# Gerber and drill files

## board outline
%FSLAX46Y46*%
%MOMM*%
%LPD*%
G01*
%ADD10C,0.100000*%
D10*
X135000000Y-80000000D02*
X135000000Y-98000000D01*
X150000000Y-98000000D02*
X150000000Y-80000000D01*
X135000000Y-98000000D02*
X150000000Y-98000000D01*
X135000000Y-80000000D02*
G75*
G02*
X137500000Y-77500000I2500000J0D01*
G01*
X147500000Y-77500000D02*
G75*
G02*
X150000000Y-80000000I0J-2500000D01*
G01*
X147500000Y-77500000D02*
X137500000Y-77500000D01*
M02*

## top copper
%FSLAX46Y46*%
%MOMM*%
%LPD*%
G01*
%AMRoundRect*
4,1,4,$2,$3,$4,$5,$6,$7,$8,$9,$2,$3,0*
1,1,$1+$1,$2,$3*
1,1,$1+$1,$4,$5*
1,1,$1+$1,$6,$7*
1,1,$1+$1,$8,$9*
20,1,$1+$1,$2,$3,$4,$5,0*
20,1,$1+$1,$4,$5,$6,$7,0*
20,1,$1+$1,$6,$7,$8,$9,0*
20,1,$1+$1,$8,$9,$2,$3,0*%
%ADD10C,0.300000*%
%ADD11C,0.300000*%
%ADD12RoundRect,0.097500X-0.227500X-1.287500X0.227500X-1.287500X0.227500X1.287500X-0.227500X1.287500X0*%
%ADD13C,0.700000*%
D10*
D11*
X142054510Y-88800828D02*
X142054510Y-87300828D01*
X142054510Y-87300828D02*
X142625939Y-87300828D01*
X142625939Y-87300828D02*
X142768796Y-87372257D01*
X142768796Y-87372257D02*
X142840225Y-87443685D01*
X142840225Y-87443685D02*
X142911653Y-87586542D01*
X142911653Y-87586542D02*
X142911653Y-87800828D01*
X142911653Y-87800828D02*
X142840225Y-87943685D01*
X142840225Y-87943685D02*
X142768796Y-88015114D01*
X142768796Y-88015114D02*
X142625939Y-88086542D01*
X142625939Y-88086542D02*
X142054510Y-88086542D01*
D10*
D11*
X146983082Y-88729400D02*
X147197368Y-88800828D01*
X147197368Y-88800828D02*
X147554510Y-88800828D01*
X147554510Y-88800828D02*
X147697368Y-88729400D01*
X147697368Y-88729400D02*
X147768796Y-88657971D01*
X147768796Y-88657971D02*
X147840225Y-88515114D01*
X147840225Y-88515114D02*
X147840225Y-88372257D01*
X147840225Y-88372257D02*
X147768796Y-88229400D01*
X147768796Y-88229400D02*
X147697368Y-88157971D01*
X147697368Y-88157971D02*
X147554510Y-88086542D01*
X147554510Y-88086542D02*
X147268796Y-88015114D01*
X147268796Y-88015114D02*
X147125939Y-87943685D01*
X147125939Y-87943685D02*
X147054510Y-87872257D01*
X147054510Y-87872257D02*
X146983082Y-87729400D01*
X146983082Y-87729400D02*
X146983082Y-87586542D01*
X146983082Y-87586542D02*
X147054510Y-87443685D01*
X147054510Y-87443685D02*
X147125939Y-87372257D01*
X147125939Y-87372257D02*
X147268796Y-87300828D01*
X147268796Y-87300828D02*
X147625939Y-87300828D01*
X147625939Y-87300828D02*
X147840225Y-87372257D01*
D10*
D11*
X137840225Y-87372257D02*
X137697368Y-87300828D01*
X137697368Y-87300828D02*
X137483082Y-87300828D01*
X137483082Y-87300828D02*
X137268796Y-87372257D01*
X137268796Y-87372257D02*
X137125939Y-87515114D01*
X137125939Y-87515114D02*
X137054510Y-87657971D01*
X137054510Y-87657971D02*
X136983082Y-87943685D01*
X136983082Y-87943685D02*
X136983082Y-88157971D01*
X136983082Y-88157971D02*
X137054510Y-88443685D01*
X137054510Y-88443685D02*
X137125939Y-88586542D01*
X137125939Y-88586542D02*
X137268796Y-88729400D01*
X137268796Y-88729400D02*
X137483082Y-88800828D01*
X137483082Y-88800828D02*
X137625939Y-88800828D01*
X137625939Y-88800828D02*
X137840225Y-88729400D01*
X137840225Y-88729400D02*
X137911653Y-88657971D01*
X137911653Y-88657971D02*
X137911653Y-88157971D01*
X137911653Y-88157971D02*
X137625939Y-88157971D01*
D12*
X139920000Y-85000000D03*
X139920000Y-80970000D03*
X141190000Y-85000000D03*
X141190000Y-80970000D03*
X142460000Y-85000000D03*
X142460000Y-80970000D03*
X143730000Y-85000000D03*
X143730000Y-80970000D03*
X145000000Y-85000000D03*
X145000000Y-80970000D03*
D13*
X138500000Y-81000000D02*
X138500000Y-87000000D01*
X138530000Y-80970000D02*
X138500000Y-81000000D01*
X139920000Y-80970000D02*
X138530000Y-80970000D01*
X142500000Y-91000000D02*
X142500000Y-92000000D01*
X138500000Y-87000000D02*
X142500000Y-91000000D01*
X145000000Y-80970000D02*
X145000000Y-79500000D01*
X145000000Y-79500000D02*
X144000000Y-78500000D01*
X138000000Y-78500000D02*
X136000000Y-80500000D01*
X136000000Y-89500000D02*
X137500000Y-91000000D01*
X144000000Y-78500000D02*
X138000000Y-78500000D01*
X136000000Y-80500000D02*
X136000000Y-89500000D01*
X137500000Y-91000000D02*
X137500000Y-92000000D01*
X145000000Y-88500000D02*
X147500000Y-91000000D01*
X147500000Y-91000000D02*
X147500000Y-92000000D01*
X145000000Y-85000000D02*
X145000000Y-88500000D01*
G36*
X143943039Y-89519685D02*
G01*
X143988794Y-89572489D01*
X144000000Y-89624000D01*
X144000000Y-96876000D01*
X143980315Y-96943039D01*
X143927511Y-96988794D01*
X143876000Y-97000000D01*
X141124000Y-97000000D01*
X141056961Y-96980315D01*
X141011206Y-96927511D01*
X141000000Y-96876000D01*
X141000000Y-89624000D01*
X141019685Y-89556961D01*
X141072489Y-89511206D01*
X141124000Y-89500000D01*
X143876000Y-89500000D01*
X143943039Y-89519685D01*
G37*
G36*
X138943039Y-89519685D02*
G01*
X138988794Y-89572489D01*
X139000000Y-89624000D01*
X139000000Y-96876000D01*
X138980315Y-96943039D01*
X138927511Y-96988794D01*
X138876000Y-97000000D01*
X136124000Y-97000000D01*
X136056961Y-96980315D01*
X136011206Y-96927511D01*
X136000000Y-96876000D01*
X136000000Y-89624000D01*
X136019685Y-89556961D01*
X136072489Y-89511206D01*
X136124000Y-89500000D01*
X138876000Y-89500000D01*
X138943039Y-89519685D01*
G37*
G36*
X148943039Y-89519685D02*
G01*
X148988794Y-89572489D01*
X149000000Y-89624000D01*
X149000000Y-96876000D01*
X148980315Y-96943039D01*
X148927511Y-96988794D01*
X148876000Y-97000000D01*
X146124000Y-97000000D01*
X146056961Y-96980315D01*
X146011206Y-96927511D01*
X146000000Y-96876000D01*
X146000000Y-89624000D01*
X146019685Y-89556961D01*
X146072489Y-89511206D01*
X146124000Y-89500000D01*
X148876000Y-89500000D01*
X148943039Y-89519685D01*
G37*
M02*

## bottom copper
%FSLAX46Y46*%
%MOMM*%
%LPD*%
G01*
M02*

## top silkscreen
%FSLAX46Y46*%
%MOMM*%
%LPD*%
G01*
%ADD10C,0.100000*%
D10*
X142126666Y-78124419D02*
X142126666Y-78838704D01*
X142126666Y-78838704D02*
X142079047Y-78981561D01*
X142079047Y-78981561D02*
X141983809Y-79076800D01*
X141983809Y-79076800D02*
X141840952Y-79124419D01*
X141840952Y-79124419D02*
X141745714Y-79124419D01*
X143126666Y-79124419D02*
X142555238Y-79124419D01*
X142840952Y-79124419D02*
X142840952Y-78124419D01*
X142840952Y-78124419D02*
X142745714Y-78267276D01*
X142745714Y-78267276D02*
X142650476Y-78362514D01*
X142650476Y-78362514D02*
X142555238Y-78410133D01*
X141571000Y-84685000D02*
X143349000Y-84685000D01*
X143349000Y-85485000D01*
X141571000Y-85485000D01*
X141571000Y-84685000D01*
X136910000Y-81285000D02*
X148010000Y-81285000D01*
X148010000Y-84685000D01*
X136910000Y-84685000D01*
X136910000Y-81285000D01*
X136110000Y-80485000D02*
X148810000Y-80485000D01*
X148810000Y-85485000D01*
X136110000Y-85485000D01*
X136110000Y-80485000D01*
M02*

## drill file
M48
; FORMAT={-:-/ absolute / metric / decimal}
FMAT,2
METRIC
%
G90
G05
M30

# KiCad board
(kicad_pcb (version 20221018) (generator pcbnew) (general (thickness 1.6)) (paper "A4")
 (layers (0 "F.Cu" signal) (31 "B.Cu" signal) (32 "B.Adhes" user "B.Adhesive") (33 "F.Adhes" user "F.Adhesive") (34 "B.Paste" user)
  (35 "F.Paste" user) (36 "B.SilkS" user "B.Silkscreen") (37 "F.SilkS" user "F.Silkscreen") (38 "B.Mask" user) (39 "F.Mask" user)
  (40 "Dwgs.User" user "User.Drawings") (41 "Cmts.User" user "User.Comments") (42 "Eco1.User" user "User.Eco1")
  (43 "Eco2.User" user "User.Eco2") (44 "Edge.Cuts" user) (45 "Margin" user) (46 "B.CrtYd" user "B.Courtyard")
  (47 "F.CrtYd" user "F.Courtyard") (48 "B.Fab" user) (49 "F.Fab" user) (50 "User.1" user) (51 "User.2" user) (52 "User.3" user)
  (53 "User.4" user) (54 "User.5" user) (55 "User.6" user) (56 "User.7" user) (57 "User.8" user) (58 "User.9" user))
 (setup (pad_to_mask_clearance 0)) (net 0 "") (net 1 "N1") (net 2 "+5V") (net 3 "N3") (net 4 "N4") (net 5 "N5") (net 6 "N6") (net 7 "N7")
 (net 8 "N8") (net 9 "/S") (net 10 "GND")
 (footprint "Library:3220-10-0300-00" (layer "F.Cu") (at 142.46 82.985)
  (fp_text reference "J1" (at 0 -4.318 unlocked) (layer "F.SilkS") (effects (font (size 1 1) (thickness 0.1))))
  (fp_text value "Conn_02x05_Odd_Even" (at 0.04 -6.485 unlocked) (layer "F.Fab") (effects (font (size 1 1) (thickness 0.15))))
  (fp_rect (start -0.889 1.7) (end 0.889 2.5) (stroke (width 0.1) (type default)) (fill none) (layer "F.SilkS"))
  (fp_rect (start 5.55 1.7) (end -5.55 -1.7) (stroke (width 0.1) (type default)) (fill none) (layer "F.SilkS"))
  (fp_rect (start 6.35 2.5) (end -6.35 -2.5) (stroke (width 0.1) (type default)) (fill none) (layer "F.SilkS"))
  (pad "1" smd roundrect (at -2.54 2.015) (size 0.65 2.77) (layers "F.Cu" "F.Paste" "F.Mask") (roundrect_rratio 0.15) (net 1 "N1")
   (thermal_bridge_angle 45))
  (pad "2" smd roundrect (at -2.54 -2.015) (size 0.65 2.77) (layers "F.Cu" "F.Paste" "F.Mask") (roundrect_rratio 0.15) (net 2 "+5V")
   (thermal_bridge_angle 45))
  (pad "3" smd roundrect (at -1.27 2.015) (size 0.65 2.77) (layers "F.Cu" "F.Paste" "F.Mask") (roundrect_rratio 0.15) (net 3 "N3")
   (thermal_bridge_angle 45))
  (pad "4" smd roundrect (at -1.27 -2.015) (size 0.65 2.77) (layers "F.Cu" "F.Paste" "F.Mask") (roundrect_rratio 0.15) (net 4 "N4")
   (thermal_bridge_angle 45))
  (pad "5" smd roundrect (at 0 2.015) (size 0.65 2.77) (layers "F.Cu" "F.Paste" "F.Mask") (roundrect_rratio 0.15) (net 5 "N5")
   (thermal_bridge_angle 45))
  (pad "6" smd roundrect (at 0 -2.015) (size 0.65 2.77) (layers "F.Cu" "F.Paste" "F.Mask") (roundrect_rratio 0.15) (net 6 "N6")
   (thermal_bridge_angle 45))
  (pad "7" smd roundrect (at 1.27 2.015) (size 0.65 2.77) (layers "F.Cu" "F.Paste" "F.Mask") (roundrect_rratio 0.15) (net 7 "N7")
   (thermal_bridge_angle 45))
  (pad "8" smd roundrect (at 1.27 -2.015) (size 0.65 2.77) (layers "F.Cu" "F.Paste" "F.Mask") (roundrect_rratio 0.15) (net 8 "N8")
   (thermal_bridge_angle 45))
  (pad "9" smd roundrect (at 2.54 2.015) (size 0.65 2.77) (layers "F.Cu" "F.Paste" "F.Mask") (roundrect_rratio 0.15) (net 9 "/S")
   (thermal_bridge_angle 45))
  (pad "10" smd roundrect (at 2.54 -2.015) (size 0.65 2.77) (layers "F.Cu" "F.Paste" "F.Mask") (roundrect_rratio 0.15) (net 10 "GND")
   (thermal_bridge_angle 45)))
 (gr_line (start 135 80) (end 135 98) (stroke (width 0.1) (type default)) (layer "Edge.Cuts"))
 (gr_line (start 150 98) (end 150 80) (stroke (width 0.1) (type default)) (layer "Edge.Cuts"))
 (gr_line (start 135 98) (end 150 98) (stroke (width 0.1) (type default)) (layer "Edge.Cuts"))
 (gr_arc (start 135 80) (mid 135.732233 78.232233) (end 137.5 77.5) (stroke (width 0.1) (type default)) (layer "Edge.Cuts"))
 (gr_arc (start 147.5 77.5) (mid 149.267767 78.232233) (end 150 80) (stroke (width 0.1) (type default)) (layer "Edge.Cuts"))
 (gr_line (start 147.5 77.5) (end 137.5 77.5) (stroke (width 0.1) (type default)) (layer "Edge.Cuts"))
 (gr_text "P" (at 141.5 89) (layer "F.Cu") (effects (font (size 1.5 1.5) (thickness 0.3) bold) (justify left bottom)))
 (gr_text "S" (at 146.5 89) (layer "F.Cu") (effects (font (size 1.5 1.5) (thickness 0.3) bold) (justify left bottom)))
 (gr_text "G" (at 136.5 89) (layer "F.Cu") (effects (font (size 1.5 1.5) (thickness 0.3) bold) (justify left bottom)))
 (segment (start 138.5 81) (end 138.5 87) (width 0.7) (layer "F.Cu") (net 2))
 (segment (start 138.53 80.97) (end 138.5 81) (width 0.7) (layer "F.Cu") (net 2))
 (segment (start 139.92 80.97) (end 138.53 80.97) (width 0.7) (layer "F.Cu") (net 2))
 (segment (start 142.5 91) (end 142.5 92) (width 0.7) (layer "F.Cu") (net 2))
 (segment (start 138.5 87) (end 142.5 91) (width 0.7) (layer "F.Cu") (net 2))
 (segment (start 145 80.97) (end 145 79.5) (width 0.7) (layer "F.Cu") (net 10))
 (segment (start 145 79.5) (end 144 78.5) (width 0.7) (layer "F.Cu") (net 10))
 (segment (start 138 78.5) (end 136 80.5) (width 0.7) (layer "F.Cu") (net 10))
 (segment (start 136 89.5) (end 137.5 91) (width 0.7) (layer "F.Cu") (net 10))
 (segment (start 144 78.5) (end 138 78.5) (width 0.7) (layer "F.Cu") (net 10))
 (segment (start 136 80.5) (end 136 89.5) (width 0.7) (layer "F.Cu") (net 10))
 (segment (start 137.5 91) (end 137.5 92) (width 0.7) (layer "F.Cu") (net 10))
 (segment (start 145 88.5) (end 147.5 91) (width 0.7) (layer "F.Cu") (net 9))
 (segment (start 147.5 91) (end 147.5 92) (width 0.7) (layer "F.Cu") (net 9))
 (segment (start 145 85) (end 145 88.5) (width 0.7) (layer "F.Cu") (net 9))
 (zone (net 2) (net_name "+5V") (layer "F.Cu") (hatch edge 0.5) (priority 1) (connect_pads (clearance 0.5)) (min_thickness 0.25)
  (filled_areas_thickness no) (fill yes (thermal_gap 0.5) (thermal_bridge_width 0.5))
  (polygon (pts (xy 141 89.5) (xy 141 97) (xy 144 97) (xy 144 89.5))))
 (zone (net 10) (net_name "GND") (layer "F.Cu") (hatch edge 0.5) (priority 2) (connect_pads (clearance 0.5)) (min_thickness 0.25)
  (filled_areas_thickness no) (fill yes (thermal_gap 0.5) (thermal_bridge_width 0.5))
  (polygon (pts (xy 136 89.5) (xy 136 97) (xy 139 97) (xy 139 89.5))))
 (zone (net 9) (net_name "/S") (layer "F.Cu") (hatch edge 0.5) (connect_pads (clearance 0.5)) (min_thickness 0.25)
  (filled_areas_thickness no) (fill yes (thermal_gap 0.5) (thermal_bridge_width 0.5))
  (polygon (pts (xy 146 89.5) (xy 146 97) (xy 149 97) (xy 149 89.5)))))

